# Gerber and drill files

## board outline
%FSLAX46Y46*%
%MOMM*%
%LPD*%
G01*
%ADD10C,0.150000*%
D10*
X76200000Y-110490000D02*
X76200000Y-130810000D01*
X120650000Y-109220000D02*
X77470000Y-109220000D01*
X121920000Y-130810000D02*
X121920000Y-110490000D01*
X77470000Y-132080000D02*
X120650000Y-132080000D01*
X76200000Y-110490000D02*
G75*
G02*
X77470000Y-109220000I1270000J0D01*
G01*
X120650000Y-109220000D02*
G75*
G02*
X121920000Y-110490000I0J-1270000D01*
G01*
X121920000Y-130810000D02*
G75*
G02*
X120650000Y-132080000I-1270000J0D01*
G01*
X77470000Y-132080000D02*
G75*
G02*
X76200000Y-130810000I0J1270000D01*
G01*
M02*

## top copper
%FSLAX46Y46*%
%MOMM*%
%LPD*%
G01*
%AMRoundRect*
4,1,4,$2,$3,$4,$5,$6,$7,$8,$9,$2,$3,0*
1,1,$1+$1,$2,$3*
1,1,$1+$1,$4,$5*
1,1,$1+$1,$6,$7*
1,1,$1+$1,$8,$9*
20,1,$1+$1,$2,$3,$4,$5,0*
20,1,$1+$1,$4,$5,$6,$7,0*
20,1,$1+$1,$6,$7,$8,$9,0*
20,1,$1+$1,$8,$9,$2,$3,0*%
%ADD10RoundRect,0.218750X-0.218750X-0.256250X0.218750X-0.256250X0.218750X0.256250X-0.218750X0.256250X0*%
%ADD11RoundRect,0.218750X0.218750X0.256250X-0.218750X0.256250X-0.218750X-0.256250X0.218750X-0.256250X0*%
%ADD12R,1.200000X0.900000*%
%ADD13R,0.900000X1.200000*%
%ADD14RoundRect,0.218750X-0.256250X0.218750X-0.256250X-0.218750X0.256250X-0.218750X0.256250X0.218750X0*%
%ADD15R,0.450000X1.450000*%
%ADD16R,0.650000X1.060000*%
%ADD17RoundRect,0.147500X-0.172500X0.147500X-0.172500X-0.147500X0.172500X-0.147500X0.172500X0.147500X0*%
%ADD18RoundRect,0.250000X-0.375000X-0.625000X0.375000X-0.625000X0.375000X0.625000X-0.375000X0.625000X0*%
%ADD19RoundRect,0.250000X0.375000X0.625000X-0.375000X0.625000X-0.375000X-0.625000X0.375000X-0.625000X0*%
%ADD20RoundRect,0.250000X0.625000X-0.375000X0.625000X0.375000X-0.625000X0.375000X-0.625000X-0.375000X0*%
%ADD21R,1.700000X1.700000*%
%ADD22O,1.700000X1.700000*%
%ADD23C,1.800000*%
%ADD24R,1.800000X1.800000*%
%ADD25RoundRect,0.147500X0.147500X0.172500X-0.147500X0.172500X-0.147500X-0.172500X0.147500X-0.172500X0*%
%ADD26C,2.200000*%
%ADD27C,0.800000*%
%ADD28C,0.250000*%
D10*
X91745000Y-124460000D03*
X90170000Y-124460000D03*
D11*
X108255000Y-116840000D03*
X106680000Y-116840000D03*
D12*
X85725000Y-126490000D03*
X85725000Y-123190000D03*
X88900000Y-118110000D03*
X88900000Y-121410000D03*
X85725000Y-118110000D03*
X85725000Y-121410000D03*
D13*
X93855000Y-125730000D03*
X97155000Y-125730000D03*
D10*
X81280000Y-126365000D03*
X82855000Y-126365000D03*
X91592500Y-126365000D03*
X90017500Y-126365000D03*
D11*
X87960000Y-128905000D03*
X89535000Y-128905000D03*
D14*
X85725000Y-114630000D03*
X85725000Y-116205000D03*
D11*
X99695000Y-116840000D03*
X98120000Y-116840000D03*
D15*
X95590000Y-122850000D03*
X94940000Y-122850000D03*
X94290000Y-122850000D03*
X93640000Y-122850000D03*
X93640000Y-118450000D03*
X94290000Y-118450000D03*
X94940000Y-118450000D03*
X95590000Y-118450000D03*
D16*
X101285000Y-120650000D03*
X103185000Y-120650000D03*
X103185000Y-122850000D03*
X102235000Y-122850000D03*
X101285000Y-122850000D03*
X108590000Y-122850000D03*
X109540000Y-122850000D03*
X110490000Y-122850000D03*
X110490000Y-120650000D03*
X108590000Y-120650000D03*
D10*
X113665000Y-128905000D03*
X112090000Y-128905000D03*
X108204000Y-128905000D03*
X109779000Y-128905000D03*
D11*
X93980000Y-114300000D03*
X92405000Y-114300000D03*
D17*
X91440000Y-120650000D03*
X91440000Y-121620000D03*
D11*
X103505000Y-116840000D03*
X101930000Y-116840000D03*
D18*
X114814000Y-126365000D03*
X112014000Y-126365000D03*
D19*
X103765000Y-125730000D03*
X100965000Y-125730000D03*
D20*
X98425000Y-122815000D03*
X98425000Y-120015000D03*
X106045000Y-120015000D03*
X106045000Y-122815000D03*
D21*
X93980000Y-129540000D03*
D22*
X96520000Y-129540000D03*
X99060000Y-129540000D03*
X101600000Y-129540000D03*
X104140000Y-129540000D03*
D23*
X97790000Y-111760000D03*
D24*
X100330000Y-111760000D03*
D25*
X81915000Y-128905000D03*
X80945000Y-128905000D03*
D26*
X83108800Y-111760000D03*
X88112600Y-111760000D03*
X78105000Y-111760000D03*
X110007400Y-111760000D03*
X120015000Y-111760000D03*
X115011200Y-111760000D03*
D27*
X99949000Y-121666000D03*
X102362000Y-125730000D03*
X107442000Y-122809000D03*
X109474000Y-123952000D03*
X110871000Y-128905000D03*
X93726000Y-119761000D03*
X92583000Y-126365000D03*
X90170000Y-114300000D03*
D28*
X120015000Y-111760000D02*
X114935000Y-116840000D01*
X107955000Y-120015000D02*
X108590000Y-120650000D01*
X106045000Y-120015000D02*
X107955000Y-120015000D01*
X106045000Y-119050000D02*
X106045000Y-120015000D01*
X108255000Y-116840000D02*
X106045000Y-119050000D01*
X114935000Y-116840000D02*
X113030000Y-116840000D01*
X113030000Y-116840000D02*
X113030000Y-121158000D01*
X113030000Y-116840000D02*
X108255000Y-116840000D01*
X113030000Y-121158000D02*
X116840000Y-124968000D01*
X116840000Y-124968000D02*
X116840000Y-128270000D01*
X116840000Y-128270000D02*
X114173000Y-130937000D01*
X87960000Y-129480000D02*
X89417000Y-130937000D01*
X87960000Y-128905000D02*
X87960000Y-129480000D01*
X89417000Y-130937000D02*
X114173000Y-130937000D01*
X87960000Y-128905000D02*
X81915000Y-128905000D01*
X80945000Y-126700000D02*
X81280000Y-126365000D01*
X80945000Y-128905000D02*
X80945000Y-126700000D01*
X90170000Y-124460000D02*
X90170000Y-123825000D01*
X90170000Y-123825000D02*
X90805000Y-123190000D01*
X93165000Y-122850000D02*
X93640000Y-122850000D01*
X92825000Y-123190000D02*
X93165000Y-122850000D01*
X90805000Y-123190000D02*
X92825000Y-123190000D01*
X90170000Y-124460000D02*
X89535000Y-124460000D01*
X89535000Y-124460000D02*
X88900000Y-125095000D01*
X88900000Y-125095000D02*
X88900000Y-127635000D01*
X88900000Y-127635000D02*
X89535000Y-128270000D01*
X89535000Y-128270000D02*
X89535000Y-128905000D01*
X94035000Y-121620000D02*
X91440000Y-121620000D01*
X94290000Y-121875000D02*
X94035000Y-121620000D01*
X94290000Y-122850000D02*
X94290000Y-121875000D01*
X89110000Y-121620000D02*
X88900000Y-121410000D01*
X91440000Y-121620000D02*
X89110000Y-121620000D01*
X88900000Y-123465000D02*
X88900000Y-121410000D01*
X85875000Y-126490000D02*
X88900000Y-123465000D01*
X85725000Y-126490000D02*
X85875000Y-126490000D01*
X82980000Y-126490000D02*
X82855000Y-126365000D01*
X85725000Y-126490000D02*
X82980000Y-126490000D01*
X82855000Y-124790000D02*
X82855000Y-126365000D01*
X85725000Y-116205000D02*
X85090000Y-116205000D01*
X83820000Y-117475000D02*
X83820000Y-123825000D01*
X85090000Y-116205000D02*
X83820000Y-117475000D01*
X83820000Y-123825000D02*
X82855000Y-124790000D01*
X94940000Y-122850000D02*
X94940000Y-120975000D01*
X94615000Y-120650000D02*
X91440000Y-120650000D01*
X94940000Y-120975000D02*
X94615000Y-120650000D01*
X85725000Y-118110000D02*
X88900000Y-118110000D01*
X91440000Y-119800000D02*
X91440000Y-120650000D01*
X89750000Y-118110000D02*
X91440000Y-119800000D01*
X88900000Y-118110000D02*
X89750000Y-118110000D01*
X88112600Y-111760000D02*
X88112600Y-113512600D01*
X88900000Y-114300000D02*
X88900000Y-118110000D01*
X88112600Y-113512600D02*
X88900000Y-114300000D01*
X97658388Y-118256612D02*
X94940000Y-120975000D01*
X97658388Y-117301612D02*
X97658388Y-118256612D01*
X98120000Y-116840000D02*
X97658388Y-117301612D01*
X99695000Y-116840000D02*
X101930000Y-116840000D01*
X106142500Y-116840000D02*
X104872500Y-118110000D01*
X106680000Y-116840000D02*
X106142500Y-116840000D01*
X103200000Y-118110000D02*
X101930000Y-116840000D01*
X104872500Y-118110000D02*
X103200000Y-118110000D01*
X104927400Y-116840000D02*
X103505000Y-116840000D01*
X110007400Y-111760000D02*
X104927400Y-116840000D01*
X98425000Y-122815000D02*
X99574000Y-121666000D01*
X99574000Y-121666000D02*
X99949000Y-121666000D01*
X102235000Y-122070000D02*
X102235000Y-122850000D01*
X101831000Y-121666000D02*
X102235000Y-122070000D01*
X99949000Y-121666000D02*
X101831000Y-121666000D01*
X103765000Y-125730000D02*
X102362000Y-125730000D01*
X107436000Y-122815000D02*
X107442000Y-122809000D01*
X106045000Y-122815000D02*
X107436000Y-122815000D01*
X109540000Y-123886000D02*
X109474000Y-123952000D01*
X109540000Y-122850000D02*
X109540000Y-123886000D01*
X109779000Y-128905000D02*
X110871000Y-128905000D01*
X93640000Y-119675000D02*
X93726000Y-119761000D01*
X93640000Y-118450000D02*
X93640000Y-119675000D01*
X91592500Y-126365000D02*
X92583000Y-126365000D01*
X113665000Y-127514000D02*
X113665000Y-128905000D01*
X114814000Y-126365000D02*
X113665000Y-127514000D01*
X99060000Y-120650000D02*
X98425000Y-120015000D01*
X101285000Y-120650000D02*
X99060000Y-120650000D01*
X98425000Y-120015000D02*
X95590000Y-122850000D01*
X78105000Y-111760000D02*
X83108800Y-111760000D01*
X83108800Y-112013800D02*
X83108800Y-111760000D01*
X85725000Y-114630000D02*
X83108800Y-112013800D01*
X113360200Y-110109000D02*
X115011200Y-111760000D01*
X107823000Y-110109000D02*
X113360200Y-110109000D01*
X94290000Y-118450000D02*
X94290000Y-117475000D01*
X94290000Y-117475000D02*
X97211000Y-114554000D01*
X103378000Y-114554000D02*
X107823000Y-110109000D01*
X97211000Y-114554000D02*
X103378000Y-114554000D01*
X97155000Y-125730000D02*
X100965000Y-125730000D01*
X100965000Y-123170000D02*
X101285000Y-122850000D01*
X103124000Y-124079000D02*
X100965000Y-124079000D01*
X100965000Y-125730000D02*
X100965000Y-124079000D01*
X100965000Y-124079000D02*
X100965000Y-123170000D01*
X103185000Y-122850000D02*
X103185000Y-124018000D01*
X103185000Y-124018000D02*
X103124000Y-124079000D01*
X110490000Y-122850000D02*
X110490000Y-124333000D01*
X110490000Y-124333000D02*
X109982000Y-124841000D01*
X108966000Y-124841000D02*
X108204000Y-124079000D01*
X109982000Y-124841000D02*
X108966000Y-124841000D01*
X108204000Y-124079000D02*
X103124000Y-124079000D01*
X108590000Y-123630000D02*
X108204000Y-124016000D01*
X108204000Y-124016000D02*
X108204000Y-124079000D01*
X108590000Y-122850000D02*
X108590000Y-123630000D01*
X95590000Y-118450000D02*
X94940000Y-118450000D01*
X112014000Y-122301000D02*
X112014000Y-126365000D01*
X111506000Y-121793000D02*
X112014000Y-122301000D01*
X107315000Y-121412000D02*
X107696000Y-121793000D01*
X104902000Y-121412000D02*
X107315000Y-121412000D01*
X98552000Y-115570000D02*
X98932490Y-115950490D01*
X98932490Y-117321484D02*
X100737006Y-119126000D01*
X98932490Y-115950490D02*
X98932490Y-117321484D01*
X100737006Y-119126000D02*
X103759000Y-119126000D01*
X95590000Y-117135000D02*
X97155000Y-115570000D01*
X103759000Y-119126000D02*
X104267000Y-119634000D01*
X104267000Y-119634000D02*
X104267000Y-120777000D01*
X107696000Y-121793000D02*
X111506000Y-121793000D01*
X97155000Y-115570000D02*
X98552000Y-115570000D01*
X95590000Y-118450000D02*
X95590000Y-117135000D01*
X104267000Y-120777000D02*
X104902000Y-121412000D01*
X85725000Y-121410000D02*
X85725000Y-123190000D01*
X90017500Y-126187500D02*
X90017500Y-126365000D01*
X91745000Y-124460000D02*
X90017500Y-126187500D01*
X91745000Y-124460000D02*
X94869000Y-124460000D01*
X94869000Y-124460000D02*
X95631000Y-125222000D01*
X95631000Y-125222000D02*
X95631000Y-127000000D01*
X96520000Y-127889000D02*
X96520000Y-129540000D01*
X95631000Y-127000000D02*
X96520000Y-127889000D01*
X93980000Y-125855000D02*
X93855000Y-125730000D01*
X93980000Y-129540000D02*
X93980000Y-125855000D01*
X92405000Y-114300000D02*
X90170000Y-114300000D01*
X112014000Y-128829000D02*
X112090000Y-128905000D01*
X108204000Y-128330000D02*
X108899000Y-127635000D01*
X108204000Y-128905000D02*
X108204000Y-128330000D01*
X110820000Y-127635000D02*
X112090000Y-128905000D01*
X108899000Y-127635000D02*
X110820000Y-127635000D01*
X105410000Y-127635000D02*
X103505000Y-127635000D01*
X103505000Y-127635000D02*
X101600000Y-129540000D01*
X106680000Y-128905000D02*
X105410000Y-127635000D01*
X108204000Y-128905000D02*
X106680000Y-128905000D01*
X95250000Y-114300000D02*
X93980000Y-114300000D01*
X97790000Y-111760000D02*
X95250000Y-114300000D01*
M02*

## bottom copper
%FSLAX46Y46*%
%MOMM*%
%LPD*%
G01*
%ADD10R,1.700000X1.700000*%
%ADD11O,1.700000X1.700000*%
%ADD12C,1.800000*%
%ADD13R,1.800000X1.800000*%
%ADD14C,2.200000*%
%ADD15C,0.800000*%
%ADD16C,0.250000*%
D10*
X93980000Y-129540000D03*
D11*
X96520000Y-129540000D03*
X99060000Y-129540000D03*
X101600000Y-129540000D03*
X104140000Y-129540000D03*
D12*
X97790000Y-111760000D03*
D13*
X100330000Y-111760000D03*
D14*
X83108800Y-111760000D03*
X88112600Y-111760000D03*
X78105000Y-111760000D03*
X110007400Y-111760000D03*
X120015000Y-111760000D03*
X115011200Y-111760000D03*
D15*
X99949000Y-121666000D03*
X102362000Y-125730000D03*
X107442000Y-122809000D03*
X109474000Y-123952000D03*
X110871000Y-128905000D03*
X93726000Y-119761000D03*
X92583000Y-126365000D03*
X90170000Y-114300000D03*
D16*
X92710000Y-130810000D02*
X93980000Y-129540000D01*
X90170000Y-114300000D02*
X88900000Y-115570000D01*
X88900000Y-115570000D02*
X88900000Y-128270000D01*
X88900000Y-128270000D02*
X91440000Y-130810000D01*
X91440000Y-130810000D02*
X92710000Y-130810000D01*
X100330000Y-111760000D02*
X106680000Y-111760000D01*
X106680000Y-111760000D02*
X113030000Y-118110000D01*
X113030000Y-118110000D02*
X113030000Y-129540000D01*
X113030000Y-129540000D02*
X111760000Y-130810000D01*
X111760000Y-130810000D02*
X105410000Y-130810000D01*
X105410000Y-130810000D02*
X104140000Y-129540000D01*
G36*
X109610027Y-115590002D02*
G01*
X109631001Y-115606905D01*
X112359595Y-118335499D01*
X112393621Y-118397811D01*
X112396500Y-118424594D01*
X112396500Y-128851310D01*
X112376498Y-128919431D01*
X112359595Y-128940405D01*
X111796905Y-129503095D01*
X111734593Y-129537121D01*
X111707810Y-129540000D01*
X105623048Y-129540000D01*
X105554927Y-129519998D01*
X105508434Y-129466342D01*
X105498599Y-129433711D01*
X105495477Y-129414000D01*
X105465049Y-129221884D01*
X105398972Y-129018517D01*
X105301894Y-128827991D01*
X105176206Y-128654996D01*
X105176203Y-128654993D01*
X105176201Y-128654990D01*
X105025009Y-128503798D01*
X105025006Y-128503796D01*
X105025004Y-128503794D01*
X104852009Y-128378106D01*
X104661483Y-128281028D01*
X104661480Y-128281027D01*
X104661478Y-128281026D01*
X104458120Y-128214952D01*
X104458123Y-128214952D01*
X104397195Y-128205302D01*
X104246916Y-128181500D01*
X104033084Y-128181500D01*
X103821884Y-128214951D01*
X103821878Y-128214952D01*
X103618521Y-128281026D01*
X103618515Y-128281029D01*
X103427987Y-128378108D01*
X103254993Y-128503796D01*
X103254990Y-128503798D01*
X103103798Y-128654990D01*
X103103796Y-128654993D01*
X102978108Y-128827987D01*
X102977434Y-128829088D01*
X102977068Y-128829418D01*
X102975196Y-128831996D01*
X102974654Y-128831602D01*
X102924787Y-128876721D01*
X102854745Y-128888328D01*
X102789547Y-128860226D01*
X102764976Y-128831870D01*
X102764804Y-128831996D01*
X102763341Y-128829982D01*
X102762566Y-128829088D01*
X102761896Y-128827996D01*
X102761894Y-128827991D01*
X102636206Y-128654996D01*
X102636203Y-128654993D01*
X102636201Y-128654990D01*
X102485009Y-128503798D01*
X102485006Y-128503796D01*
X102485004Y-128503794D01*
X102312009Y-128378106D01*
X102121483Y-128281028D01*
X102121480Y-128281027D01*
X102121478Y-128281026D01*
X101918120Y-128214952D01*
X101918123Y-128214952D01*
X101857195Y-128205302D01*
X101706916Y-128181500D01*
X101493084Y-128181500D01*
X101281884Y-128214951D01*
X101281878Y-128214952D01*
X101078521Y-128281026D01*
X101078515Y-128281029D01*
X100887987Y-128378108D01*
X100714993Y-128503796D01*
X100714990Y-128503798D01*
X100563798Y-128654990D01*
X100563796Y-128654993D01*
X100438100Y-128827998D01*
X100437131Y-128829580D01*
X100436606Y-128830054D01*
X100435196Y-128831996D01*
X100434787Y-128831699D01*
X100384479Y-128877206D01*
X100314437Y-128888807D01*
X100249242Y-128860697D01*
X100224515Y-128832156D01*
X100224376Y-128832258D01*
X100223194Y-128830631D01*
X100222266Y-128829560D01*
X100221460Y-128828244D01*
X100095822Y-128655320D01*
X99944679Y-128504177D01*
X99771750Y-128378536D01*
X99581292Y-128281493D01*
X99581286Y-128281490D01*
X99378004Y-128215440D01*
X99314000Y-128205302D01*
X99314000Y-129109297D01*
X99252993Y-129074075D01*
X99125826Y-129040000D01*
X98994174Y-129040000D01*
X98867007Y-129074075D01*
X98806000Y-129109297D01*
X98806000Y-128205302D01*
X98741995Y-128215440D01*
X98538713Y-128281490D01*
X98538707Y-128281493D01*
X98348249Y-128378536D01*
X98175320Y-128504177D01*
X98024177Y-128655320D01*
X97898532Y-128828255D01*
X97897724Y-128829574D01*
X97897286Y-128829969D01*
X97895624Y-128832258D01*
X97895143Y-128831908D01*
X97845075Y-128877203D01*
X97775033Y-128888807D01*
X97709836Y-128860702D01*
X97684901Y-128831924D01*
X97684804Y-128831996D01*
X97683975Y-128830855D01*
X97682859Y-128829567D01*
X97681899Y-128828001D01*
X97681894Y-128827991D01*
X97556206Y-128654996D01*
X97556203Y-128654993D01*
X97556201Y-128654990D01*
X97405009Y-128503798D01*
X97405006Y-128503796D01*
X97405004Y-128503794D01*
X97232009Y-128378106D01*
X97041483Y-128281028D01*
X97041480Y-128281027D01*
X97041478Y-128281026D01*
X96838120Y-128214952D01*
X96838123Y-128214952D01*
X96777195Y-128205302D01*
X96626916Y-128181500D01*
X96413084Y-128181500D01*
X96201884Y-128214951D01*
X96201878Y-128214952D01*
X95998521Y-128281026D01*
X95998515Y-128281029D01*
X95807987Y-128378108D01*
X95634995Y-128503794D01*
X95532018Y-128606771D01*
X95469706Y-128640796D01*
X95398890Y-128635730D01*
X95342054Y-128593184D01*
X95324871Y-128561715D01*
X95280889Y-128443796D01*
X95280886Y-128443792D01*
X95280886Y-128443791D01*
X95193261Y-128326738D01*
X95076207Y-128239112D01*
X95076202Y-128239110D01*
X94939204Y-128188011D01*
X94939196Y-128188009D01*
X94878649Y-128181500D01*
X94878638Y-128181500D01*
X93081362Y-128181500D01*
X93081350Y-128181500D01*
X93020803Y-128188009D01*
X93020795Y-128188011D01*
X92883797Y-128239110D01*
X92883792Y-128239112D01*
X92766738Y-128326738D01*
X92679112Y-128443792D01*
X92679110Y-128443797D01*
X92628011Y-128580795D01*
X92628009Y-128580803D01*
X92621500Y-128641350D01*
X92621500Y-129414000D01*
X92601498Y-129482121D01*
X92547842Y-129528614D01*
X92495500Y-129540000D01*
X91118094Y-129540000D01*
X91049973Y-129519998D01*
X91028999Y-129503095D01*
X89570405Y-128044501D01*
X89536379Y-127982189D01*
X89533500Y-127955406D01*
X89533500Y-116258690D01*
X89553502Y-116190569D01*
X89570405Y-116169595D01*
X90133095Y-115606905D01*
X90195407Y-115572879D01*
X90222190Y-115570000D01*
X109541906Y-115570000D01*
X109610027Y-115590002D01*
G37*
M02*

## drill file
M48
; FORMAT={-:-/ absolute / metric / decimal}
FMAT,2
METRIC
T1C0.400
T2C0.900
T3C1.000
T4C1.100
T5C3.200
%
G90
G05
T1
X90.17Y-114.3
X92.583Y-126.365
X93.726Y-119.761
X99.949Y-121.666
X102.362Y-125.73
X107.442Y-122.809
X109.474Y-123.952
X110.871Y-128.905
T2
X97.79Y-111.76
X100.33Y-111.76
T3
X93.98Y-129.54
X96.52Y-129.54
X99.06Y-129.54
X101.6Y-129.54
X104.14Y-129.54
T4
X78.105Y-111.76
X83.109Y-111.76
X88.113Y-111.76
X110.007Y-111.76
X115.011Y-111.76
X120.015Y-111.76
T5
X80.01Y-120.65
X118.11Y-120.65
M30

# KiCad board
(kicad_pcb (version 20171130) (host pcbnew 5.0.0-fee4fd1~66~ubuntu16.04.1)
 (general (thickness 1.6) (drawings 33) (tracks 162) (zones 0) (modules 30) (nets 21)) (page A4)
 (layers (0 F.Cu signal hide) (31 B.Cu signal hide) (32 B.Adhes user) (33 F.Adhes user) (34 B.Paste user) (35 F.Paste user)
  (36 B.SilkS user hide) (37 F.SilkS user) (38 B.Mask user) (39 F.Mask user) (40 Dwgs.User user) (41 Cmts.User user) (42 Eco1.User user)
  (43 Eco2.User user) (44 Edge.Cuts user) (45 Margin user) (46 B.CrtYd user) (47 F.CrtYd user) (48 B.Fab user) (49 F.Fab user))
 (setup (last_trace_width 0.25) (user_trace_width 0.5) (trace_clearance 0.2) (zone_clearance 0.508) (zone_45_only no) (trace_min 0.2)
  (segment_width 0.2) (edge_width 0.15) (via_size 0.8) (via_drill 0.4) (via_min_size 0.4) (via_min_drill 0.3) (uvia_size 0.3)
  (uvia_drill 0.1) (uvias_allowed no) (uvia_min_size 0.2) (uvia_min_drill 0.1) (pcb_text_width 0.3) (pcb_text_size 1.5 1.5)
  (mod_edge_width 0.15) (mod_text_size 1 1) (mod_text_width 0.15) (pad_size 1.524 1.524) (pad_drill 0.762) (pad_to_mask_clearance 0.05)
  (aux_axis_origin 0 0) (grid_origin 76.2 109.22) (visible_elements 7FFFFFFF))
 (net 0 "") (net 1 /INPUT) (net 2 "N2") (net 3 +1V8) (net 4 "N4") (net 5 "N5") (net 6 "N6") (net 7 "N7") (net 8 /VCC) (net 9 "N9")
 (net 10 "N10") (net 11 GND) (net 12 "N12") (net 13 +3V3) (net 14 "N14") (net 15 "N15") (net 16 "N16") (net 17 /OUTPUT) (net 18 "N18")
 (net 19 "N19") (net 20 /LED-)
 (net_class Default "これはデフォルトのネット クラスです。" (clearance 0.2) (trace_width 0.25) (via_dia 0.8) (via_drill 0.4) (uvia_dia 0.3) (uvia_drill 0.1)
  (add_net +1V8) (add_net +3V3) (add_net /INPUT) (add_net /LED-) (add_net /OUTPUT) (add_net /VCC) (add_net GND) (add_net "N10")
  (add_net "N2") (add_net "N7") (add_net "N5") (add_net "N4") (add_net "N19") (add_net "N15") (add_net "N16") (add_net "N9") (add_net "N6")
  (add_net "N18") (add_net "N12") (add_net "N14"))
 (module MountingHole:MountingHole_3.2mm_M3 (layer F.Cu) (at 80.01 120.65)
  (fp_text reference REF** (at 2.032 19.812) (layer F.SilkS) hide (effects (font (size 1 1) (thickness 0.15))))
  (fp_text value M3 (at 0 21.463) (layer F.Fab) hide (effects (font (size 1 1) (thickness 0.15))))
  (pad 1 np_thru_hole circle (at 0 0) (size 3.2 3.2) (drill 3.2) (layers *.Cu *.Mask)))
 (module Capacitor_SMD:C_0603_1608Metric (layer F.Cu) (at 90.9575 124.46)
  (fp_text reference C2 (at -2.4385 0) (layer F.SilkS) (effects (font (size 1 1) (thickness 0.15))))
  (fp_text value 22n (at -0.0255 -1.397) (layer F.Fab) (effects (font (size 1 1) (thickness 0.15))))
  (pad 2 smd roundrect (at 0.7875 0) (size 0.875 0.95) (layers F.Cu F.Paste F.Mask) (roundrect_rratio 0.25) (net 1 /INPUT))
  (pad 1 smd roundrect (at -0.7875 0) (size 0.875 0.95) (layers F.Cu F.Paste F.Mask) (roundrect_rratio 0.25) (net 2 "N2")))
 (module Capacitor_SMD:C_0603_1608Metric (layer F.Cu) (at 107.4675 116.84 180)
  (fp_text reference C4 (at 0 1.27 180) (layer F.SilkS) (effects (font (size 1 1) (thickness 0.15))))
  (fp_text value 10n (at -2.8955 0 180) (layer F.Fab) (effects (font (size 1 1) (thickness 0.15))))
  (pad 1 smd roundrect (at -0.7875 0 180) (size 0.875 0.95) (layers F.Cu F.Paste F.Mask) (roundrect_rratio 0.25) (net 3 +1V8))
  (pad 2 smd roundrect (at 0.7875 0 180) (size 0.875 0.95) (layers F.Cu F.Paste F.Mask) (roundrect_rratio 0.25) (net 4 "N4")))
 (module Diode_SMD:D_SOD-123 (layer F.Cu) (at 85.725 124.84 90)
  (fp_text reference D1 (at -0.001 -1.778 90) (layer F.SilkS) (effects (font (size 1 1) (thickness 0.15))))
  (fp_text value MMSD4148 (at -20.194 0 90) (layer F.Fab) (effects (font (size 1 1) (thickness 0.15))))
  (pad 1 smd rect (at -1.65 0 90) (size 0.9 1.2) (layers F.Cu F.Paste F.Mask) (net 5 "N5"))
  (pad 2 smd rect (at 1.65 0 90) (size 0.9 1.2) (layers F.Cu F.Paste F.Mask) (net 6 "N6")))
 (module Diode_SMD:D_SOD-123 (layer F.Cu) (at 88.9 119.76 270)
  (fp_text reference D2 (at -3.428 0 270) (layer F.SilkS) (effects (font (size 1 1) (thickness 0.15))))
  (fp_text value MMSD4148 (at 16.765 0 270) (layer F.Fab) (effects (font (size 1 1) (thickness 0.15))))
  (pad 1 smd rect (at -1.65 0 270) (size 0.9 1.2) (layers F.Cu F.Paste F.Mask) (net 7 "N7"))
  (pad 2 smd rect (at 1.65 0 270) (size 0.9 1.2) (layers F.Cu F.Paste F.Mask) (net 5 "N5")))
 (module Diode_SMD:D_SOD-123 (layer F.Cu) (at 85.725 119.76 90)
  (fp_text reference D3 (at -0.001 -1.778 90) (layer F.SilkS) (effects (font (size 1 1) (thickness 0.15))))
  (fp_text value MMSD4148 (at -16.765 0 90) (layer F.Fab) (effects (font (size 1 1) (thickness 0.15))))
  (pad 2 smd rect (at 1.65 0 90) (size 0.9 1.2) (layers F.Cu F.Paste F.Mask) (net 7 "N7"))
  (pad 1 smd rect (at -1.65 0 90) (size 0.9 1.2) (layers F.Cu F.Paste F.Mask) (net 6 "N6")))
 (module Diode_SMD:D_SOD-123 (layer F.Cu) (at 95.505 125.73 180)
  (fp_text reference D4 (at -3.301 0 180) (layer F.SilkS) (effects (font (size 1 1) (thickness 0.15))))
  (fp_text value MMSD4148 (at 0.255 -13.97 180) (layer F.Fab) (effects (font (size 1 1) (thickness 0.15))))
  (pad 2 smd rect (at 1.65 0 180) (size 0.9 1.2) (layers F.Cu F.Paste F.Mask) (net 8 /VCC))
  (pad 1 smd rect (at -1.65 0 180) (size 0.9 1.2) (layers F.Cu F.Paste F.Mask) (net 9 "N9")))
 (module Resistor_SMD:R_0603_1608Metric (layer F.Cu) (at 82.0675 126.365)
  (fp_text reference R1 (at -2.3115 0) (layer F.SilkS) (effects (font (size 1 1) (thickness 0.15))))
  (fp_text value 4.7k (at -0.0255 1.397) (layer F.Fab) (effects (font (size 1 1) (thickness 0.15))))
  (pad 1 smd roundrect (at -0.7875 0) (size 0.875 0.95) (layers F.Cu F.Paste F.Mask) (roundrect_rratio 0.25) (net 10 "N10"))
  (pad 2 smd roundrect (at 0.7875 0) (size 0.875 0.95) (layers F.Cu F.Paste F.Mask) (roundrect_rratio 0.25) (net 5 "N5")))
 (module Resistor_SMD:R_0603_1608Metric (layer F.Cu) (at 90.805 126.365)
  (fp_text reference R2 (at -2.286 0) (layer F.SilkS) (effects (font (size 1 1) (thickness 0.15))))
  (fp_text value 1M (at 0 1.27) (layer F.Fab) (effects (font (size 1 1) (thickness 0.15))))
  (pad 2 smd roundrect (at 0.7875 0) (size 0.875 0.95) (layers F.Cu F.Paste F.Mask) (roundrect_rratio 0.25) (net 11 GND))
  (pad 1 smd roundrect (at -0.7875 0) (size 0.875 0.95) (layers F.Cu F.Paste F.Mask) (roundrect_rratio 0.25) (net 1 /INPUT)))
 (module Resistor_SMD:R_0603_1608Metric (layer F.Cu) (at 88.7475 128.905 180)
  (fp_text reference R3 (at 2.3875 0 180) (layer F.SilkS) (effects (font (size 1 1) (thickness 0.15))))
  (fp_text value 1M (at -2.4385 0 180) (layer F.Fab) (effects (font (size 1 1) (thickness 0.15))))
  (pad 2 smd roundrect (at 0.7875 0 180) (size 0.875 0.95) (layers F.Cu F.Paste F.Mask) (roundrect_rratio 0.25) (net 3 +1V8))
  (pad 1 smd roundrect (at -0.7875 0 180) (size 0.875 0.95) (layers F.Cu F.Paste F.Mask) (roundrect_rratio 0.25) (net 2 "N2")))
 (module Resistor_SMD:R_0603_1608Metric (layer F.Cu) (at 85.725 115.4175 270)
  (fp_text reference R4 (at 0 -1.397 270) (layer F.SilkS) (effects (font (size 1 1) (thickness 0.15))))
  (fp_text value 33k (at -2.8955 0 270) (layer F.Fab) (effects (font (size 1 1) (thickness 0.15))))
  (pad 1 smd roundrect (at -0.7875 0 270) (size 0.875 0.95) (layers F.Cu F.Paste F.Mask) (roundrect_rratio 0.25) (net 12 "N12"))
  (pad 2 smd roundrect (at 0.7875 0 270) (size 0.875 0.95) (layers F.Cu F.Paste F.Mask) (roundrect_rratio 0.25) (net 5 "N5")))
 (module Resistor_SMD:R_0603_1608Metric (layer F.Cu) (at 98.9075 116.84 180)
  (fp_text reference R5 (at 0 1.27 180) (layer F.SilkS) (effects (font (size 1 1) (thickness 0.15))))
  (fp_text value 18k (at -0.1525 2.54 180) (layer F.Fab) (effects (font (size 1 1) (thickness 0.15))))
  (pad 1 smd roundrect (at -0.7875 0 180) (size 0.875 0.95) (layers F.Cu F.Paste F.Mask) (roundrect_rratio 0.25) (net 4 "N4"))
  (pad 2 smd roundrect (at 0.7875 0 180) (size 0.875 0.95) (layers F.Cu F.Paste F.Mask) (roundrect_rratio 0.25) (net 7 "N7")))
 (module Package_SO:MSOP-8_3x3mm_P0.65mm (layer F.Cu) (at 94.615 120.65 270)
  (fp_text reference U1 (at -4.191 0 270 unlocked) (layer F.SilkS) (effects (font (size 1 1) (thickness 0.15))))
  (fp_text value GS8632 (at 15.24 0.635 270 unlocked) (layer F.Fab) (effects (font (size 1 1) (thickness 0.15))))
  (pad 8 smd rect (at 2.2 -0.975 270) (size 1.45 0.45) (layers F.Cu F.Paste F.Mask) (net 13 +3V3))
  (pad 7 smd rect (at 2.2 -0.325 270) (size 1.45 0.45) (layers F.Cu F.Paste F.Mask) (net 7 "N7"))
  (pad 6 smd rect (at 2.2 0.325 270) (size 1.45 0.45) (layers F.Cu F.Paste F.Mask) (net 5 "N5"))
  (pad 5 smd rect (at 2.2 0.975 270) (size 1.45 0.45) (layers F.Cu F.Paste F.Mask) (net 2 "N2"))
  (pad 4 smd rect (at -2.2 0.975 270) (size 1.45 0.45) (layers F.Cu F.Paste F.Mask) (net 11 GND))
  (pad 3 smd rect (at -2.2 0.325 270) (size 1.45 0.45) (layers F.Cu F.Paste F.Mask) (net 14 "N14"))
  (pad 2 smd rect (at -2.2 -0.325 270) (size 1.45 0.45) (layers F.Cu F.Paste F.Mask) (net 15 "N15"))
  (pad 1 smd rect (at -2.2 -0.975 270) (size 1.45 0.45) (layers F.Cu F.Paste F.Mask) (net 15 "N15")))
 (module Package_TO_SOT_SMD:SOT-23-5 (layer F.Cu) (at 102.235 121.75 90)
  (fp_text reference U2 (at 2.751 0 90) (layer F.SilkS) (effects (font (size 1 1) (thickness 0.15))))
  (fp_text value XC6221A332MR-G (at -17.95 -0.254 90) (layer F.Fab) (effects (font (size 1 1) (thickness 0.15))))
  (pad 5 smd rect (at 1.1 -0.95 90) (size 1.06 0.65) (layers F.Cu F.Paste F.Mask) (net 13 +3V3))
  (pad 4 smd rect (at 1.1 0.95 90) (size 1.06 0.65) (layers F.Cu F.Paste F.Mask))
  (pad 3 smd rect (at -1.1 0.95 90) (size 1.06 0.65) (layers F.Cu F.Paste F.Mask) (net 9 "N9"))
  (pad 2 smd rect (at -1.1 0 90) (size 1.06 0.65) (layers F.Cu F.Paste F.Mask) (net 11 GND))
  (pad 1 smd rect (at -1.1 -0.95 90) (size 1.06 0.65) (layers F.Cu F.Paste F.Mask) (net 9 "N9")))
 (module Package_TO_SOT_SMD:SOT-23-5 (layer F.Cu) (at 109.54 121.75 90)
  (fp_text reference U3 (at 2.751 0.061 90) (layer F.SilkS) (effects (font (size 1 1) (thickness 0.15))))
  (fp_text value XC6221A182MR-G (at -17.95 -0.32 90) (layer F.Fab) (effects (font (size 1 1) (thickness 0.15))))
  (pad 1 smd rect (at -1.1 -0.95 90) (size 1.06 0.65) (layers F.Cu F.Paste F.Mask) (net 9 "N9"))
  (pad 2 smd rect (at -1.1 0 90) (size 1.06 0.65) (layers F.Cu F.Paste F.Mask) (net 11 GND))
  (pad 3 smd rect (at -1.1 0.95 90) (size 1.06 0.65) (layers F.Cu F.Paste F.Mask) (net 9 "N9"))
  (pad 4 smd rect (at 1.1 0.95 90) (size 1.06 0.65) (layers F.Cu F.Paste F.Mask))
  (pad 5 smd rect (at 1.1 -0.95 90) (size 1.06 0.65) (layers F.Cu F.Paste F.Mask) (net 3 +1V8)))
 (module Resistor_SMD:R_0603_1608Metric (layer F.Cu) (at 112.8775 128.905)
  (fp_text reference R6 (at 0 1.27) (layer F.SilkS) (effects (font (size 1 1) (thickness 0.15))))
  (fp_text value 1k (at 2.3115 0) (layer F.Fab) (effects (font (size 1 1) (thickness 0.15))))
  (pad 2 smd roundrect (at 0.7875 0) (size 0.875 0.95) (layers F.Cu F.Paste F.Mask) (roundrect_rratio 0.25) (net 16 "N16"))
  (pad 1 smd roundrect (at -0.7875 0) (size 0.875 0.95) (layers F.Cu F.Paste F.Mask) (roundrect_rratio 0.25) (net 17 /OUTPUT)))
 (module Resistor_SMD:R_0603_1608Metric (layer F.Cu) (at 108.9915 128.905)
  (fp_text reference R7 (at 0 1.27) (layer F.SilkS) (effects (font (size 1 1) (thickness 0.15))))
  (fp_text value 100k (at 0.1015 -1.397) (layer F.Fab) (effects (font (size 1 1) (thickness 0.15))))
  (pad 1 smd roundrect (at -0.7875 0) (size 0.875 0.95) (layers F.Cu F.Paste F.Mask) (roundrect_rratio 0.25) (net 17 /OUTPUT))
  (pad 2 smd roundrect (at 0.7875 0) (size 0.875 0.95) (layers F.Cu F.Paste F.Mask) (roundrect_rratio 0.25) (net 11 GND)))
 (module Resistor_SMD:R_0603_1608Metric (layer F.Cu) (at 93.1925 114.3 180)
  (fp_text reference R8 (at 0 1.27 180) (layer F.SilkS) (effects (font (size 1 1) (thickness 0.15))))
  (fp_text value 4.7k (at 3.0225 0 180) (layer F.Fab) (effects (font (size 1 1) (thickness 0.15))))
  (pad 1 smd roundrect (at -0.7875 0 180) (size 0.875 0.95) (layers F.Cu F.Paste F.Mask) (roundrect_rratio 0.25) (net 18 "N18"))
  (pad 2 smd roundrect (at 0.7875 0 180) (size 0.875 0.95) (layers F.Cu F.Paste F.Mask) (roundrect_rratio 0.25) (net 8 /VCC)))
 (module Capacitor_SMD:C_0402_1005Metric (layer F.Cu) (at 91.44 121.135 270)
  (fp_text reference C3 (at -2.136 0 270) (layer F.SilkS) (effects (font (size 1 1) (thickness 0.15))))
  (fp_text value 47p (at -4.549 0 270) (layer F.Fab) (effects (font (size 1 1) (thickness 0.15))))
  (pad 1 smd roundrect (at -0.485 0 270) (size 0.59 0.64) (layers F.Cu F.Paste F.Mask) (roundrect_rratio 0.25) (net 7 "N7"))
  (pad 2 smd roundrect (at 0.485 0 270) (size 0.59 0.64) (layers F.Cu F.Paste F.Mask) (roundrect_rratio 0.25) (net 5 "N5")))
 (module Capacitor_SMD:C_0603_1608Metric (layer F.Cu) (at 102.7175 116.84 180)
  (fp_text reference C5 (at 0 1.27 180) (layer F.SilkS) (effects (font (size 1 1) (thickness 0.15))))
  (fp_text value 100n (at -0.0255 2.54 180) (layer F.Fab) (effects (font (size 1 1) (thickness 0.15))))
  (pad 1 smd roundrect (at -0.7875 0 180) (size 0.875 0.95) (layers F.Cu F.Paste F.Mask) (roundrect_rratio 0.25) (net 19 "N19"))
  (pad 2 smd roundrect (at 0.7875 0 180) (size 0.875 0.95) (layers F.Cu F.Paste F.Mask) (roundrect_rratio 0.25) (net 4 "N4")))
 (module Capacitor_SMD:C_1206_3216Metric (layer F.Cu) (at 113.414 126.365)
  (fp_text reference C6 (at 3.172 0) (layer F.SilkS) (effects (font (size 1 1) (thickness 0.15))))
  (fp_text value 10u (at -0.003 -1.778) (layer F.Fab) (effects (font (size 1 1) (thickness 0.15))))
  (pad 2 smd roundrect (at 1.4 0) (size 1.25 1.75) (layers F.Cu F.Paste F.Mask) (roundrect_rratio 0.2) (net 16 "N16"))
  (pad 1 smd roundrect (at -1.4 0) (size 1.25 1.75) (layers F.Cu F.Paste F.Mask) (roundrect_rratio 0.2) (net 15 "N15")))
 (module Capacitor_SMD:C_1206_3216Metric (layer F.Cu) (at 102.365 125.73 180)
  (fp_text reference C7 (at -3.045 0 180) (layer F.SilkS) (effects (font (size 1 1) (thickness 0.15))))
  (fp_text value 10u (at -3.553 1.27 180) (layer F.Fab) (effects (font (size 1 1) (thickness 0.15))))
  (pad 1 smd roundrect (at -1.4 0 180) (size 1.25 1.75) (layers F.Cu F.Paste F.Mask) (roundrect_rratio 0.2) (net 11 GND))
  (pad 2 smd roundrect (at 1.4 0 180) (size 1.25 1.75) (layers F.Cu F.Paste F.Mask) (roundrect_rratio 0.2) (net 9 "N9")))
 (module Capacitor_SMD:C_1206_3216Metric (layer F.Cu) (at 98.425 121.415 90)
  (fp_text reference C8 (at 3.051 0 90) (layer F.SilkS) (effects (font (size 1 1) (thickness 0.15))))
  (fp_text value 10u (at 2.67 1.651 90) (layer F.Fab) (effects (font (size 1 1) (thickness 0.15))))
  (pad 1 smd roundrect (at -1.4 0 90) (size 1.25 1.75) (layers F.Cu F.Paste F.Mask) (roundrect_rratio 0.2) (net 11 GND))
  (pad 2 smd roundrect (at 1.4 0 90) (size 1.25 1.75) (layers F.Cu F.Paste F.Mask) (roundrect_rratio 0.2) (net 13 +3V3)))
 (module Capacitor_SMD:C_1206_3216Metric (layer F.Cu) (at 106.045 121.415 90)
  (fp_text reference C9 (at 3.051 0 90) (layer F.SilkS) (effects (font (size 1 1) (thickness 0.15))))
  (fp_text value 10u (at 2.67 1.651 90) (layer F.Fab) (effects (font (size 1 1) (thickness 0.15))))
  (pad 2 smd roundrect (at 1.4 0 90) (size 1.25 1.75) (layers F.Cu F.Paste F.Mask) (roundrect_rratio 0.2) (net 3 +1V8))
  (pad 1 smd roundrect (at -1.4 0 90) (size 1.25 1.75) (layers F.Cu F.Paste F.Mask) (roundrect_rratio 0.2) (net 11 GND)))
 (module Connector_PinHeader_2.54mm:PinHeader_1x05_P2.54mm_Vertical (layer F.Cu) (at 93.98 129.54 90)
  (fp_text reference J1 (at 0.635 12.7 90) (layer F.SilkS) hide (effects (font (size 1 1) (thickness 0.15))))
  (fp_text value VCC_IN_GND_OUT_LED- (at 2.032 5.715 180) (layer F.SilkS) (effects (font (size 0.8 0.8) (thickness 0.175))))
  (pad 1 thru_hole rect (at 0 0 90) (size 1.7 1.7) (drill 1) (layers *.Cu *.Mask) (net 8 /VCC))
  (pad 2 thru_hole oval (at 0 2.54 90) (size 1.7 1.7) (drill 1) (layers *.Cu *.Mask) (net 1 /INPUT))
  (pad 3 thru_hole oval (at 0 5.08 90) (size 1.7 1.7) (drill 1) (layers *.Cu *.Mask) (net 11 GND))
  (pad 4 thru_hole oval (at 0 7.62 90) (size 1.7 1.7) (drill 1) (layers *.Cu *.Mask) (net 17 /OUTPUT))
  (pad 5 thru_hole oval (at 0 10.16 90) (size 1.7 1.7) (drill 1) (layers *.Cu *.Mask) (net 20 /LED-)))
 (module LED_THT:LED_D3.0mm (layer F.Cu) (at 100.33 111.76 180)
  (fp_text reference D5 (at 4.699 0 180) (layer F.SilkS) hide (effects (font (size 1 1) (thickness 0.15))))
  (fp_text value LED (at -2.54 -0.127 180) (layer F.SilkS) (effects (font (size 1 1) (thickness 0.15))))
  (pad 2 thru_hole circle (at 2.54 0 180) (size 1.8 1.8) (drill 0.9) (layers *.Cu *.Mask) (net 18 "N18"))
  (pad 1 thru_hole rect (at 0 0 180) (size 1.8 1.8) (drill 0.9) (layers *.Cu *.Mask) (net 20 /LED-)))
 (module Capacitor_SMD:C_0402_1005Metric (layer F.Cu) (at 81.43 128.905 180)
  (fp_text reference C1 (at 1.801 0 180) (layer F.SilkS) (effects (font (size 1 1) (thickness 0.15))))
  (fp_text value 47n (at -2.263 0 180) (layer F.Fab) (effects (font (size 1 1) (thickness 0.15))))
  (pad 1 smd roundrect (at -0.485 0 180) (size 0.59 0.64) (layers F.Cu F.Paste F.Mask) (roundrect_rratio 0.25) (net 3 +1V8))
  (pad 2 smd roundrect (at 0.485 0 180) (size 0.59 0.64) (layers F.Cu F.Paste F.Mask) (roundrect_rratio 0.25) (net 10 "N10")))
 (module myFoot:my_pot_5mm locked (layer F.Cu) (at 83.1088 111.76 180)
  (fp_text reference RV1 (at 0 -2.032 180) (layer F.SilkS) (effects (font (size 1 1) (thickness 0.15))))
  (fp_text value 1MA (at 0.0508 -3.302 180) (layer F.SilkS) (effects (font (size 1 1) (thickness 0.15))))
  (pad 2 thru_hole circle (at 0 0 180) (size 2.2 2.2) (drill 1.1) (layers *.Cu *.Mask) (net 12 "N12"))
  (pad 1 thru_hole circle (at -5.0038 0 180) (size 2.2 2.2) (drill 1.1) (layers *.Cu *.Mask) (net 7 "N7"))
  (pad 3 thru_hole circle (at 5.0038 0 180) (size 2.2 2.2) (drill 1.1) (layers *.Cu *.Mask) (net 12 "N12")))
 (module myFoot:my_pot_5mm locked (layer F.Cu) (at 115.0112 111.76 180)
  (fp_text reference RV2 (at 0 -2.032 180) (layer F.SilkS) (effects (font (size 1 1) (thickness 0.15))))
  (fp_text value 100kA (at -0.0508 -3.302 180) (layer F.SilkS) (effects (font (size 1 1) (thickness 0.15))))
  (pad 3 thru_hole circle (at 5.0038 0 180) (size 2.2 2.2) (drill 1.1) (layers *.Cu *.Mask) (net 19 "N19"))
  (pad 1 thru_hole circle (at -5.0038 0 180) (size 2.2 2.2) (drill 1.1) (layers *.Cu *.Mask) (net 3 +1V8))
  (pad 2 thru_hole circle (at 0 0 180) (size 2.2 2.2) (drill 1.1) (layers *.Cu *.Mask) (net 14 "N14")))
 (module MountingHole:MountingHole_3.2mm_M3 (layer F.Cu) (at 118.11 120.65)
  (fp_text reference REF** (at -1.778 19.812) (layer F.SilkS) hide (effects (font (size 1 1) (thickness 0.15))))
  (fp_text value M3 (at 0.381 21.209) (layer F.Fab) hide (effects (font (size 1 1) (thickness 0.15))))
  (pad 1 np_thru_hole circle (at 0 0) (size 3.2 3.2) (drill 3.2) (layers *.Cu *.Mask)))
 (gr_line (start 76.2 110.49) (end 76.2 130.81) (layer Edge.Cuts) (width 0.15))
 (gr_line (start 120.65 109.22) (end 77.47 109.22) (layer Edge.Cuts) (width 0.15))
 (gr_line (start 121.92 130.81) (end 121.92 110.49) (layer Edge.Cuts) (width 0.15))
 (gr_line (start 77.47 132.08) (end 120.65 132.08) (layer Edge.Cuts) (width 0.15))
 (gr_arc (start 77.47 110.49) (end 77.47 109.22) (angle -90) (layer Edge.Cuts) (width 0.15))
 (gr_arc (start 120.65 110.49) (end 121.92 110.49) (angle -90) (layer Edge.Cuts) (width 0.15))
 (gr_arc (start 120.65 130.81) (end 120.65 132.08) (angle -90) (layer Edge.Cuts) (width 0.15))
 (gr_arc (start 77.47 130.81) (end 76.2 130.81) (angle -90) (layer Edge.Cuts) (width 0.15))
 (segment (start 120.015 111.76) (end 114.935 116.84) (width 0.25) (layer F.Cu) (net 3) (status 10))
 (segment (start 107.955 120.015) (end 108.59 120.65) (width 0.25) (layer F.Cu) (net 3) (status 20))
 (segment (start 106.045 120.015) (end 107.955 120.015) (width 0.25) (layer F.Cu) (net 3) (status 10))
 (segment (start 106.045 119.05) (end 106.045 120.015) (width 0.25) (layer F.Cu) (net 3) (status 20))
 (segment (start 108.255 116.84) (end 106.045 119.05) (width 0.25) (layer F.Cu) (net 3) (status 10))
 (segment (start 114.935 116.84) (end 113.03 116.84) (width 0.25) (layer F.Cu) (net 3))
 (segment (start 113.03 116.84) (end 113.03 121.158) (width 0.25) (layer F.Cu) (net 3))
 (segment (start 113.03 116.84) (end 108.255 116.84) (width 0.25) (layer F.Cu) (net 3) (status 20))
 (segment (start 113.03 121.158) (end 116.84 124.968) (width 0.25) (layer F.Cu) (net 3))
 (segment (start 116.84 124.968) (end 116.84 128.27) (width 0.25) (layer F.Cu) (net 3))
 (segment (start 116.84 128.27) (end 114.173 130.937) (width 0.25) (layer F.Cu) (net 3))
 (segment (start 87.96 129.48) (end 89.417 130.937) (width 0.25) (layer F.Cu) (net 3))
 (segment (start 87.96 128.905) (end 87.96 129.48) (width 0.25) (layer F.Cu) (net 3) (status 10))
 (segment (start 89.417 130.937) (end 114.173 130.937) (width 0.25) (layer F.Cu) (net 3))
 (segment (start 87.96 128.905) (end 81.915 128.905) (width 0.25) (layer F.Cu) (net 3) (status 30))
 (segment (start 80.945 126.7) (end 81.28 126.365) (width 0.25) (layer F.Cu) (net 10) (status 30))
 (segment (start 80.945 128.905) (end 80.945 126.7) (width 0.25) (layer F.Cu) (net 10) (status 30))
 (segment (start 90.17 124.46) (end 90.17 123.825) (width 0.25) (layer F.Cu) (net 2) (status 10))
 (segment (start 90.17 123.825) (end 90.805 123.19) (width 0.25) (layer F.Cu) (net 2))
 (segment (start 93.165 122.85) (end 93.64 122.85) (width 0.25) (layer F.Cu) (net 2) (status 20))
 (segment (start 92.825 123.19) (end 93.165 122.85) (width 0.25) (layer F.Cu) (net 2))
 (segment (start 90.805 123.19) (end 92.825 123.19) (width 0.25) (layer F.Cu) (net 2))
 (segment (start 90.17 124.46) (end 89.535 124.46) (width 0.25) (layer F.Cu) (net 2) (status 10))
 (segment (start 89.535 124.46) (end 88.9 125.095) (width 0.25) (layer F.Cu) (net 2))
 (segment (start 88.9 125.095) (end 88.9 127.635) (width 0.25) (layer F.Cu) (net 2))
 (segment (start 88.9 127.635) (end 89.535 128.27) (width 0.25) (layer F.Cu) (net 2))
 (segment (start 89.535 128.27) (end 89.535 128.905) (width 0.25) (layer F.Cu) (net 2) (status 20))
 (segment (start 94.035 121.62) (end 91.44 121.62) (width 0.25) (layer F.Cu) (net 5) (status 20))
 (segment (start 94.29 121.875) (end 94.035 121.62) (width 0.25) (layer F.Cu) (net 5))
 (segment (start 94.29 122.85) (end 94.29 121.875) (width 0.25) (layer F.Cu) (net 5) (status 10))
 (segment (start 89.11 121.62) (end 88.9 121.41) (width 0.25) (layer F.Cu) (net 5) (status 30))
 (segment (start 91.44 121.62) (end 89.11 121.62) (width 0.25) (layer F.Cu) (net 5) (status 30))
 (segment (start 88.9 123.465) (end 88.9 121.41) (width 0.25) (layer F.Cu) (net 5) (status 20))
 (segment (start 85.875 126.49) (end 88.9 123.465) (width 0.25) (layer F.Cu) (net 5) (status 10))
 (segment (start 85.725 126.49) (end 85.875 126.49) (width 0.25) (layer F.Cu) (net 5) (status 30))
 (segment (start 82.98 126.49) (end 82.855 126.365) (width 0.25) (layer F.Cu) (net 5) (status 30))
 (segment (start 85.725 126.49) (end 82.98 126.49) (width 0.25) (layer F.Cu) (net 5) (status 30))
 (segment (start 82.855 124.79) (end 82.855 126.365) (width 0.25) (layer F.Cu) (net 5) (status 20))
 (segment (start 85.725 116.205) (end 85.09 116.205) (width 0.25) (layer F.Cu) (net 5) (status 10))
 (segment (start 83.82 117.475) (end 83.82 123.825) (width 0.25) (layer F.Cu) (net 5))
 (segment (start 85.09 116.205) (end 83.82 117.475) (width 0.25) (layer F.Cu) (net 5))
 (segment (start 83.82 123.825) (end 82.855 124.79) (width 0.25) (layer F.Cu) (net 5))
 (segment (start 94.94 122.85) (end 94.94 120.975) (width 0.25) (layer F.Cu) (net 7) (status 10))
 (segment (start 94.615 120.65) (end 91.44 120.65) (width 0.25) (layer F.Cu) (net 7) (status 20))
 (segment (start 94.94 120.975) (end 94.615 120.65) (width 0.25) (layer F.Cu) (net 7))
 (segment (start 85.725 118.11) (end 88.9 118.11) (width 0.25) (layer F.Cu) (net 7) (status 30))
 (segment (start 91.44 119.8) (end 91.44 120.65) (width 0.25) (layer F.Cu) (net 7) (status 20))
 (segment (start 89.75 118.11) (end 91.44 119.8) (width 0.25) (layer F.Cu) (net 7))
 (segment (start 88.9 118.11) (end 89.75 118.11) (width 0.25) (layer F.Cu) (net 7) (status 10))
 (segment (start 88.1126 111.76) (end 88.1126 113.5126) (width 0.25) (layer F.Cu) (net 7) (status 10))
 (segment (start 88.9 114.3) (end 88.9 118.11) (width 0.25) (layer F.Cu) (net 7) (status 20))
 (segment (start 88.1126 113.5126) (end 88.9 114.3) (width 0.25) (layer F.Cu) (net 7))
 (segment (start 97.658388 118.256612) (end 94.94 120.975) (width 0.25) (layer F.Cu) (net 7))
 (segment (start 97.658388 117.301612) (end 97.658388 118.256612) (width 0.25) (layer F.Cu) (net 7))
 (segment (start 98.12 116.84) (end 97.658388 117.301612) (width 0.25) (layer F.Cu) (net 7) (status 10))
 (segment (start 99.695 116.84) (end 101.93 116.84) (width 0.25) (layer F.Cu) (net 4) (status 30))
 (segment (start 106.1425 116.84) (end 104.8725 118.11) (width 0.25) (layer F.Cu) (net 4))
 (segment (start 106.68 116.84) (end 106.1425 116.84) (width 0.25) (layer F.Cu) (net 4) (status 10))
 (segment (start 103.2 118.11) (end 101.93 116.84) (width 0.25) (layer F.Cu) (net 4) (status 20))
 (segment (start 104.8725 118.11) (end 103.2 118.11) (width 0.25) (layer F.Cu) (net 4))
 (segment (start 104.9274 116.84) (end 103.505 116.84) (width 0.25) (layer F.Cu) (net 19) (status 20))
 (segment (start 110.0074 111.76) (end 104.9274 116.84) (width 0.25) (layer F.Cu) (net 19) (status 10))
 (segment (start 98.425 122.815) (end 99.574 121.666) (width 0.25) (layer F.Cu) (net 11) (status 10))
 (via (at 99.949 121.666) (size 0.8) (drill 0.4) (layers F.Cu B.Cu) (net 11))
 (segment (start 99.574 121.666) (end 99.949 121.666) (width 0.25) (layer F.Cu) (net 11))
 (segment (start 102.235 122.07) (end 102.235 122.85) (width 0.25) (layer F.Cu) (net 11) (status 20))
 (segment (start 101.831 121.666) (end 102.235 122.07) (width 0.25) (layer F.Cu) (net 11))
 (segment (start 99.949 121.666) (end 101.831 121.666) (width 0.25) (layer F.Cu) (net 11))
 (via (at 102.362 125.73) (size 0.8) (drill 0.4) (layers F.Cu B.Cu) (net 11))
 (segment (start 103.765 125.73) (end 102.362 125.73) (width 0.25) (layer F.Cu) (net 11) (status 10))
 (via (at 107.442 122.809) (size 0.8) (drill 0.4) (layers F.Cu B.Cu) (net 11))
 (segment (start 107.436 122.815) (end 107.442 122.809) (width 0.25) (layer F.Cu) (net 11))
 (segment (start 106.045 122.815) (end 107.436 122.815) (width 0.25) (layer F.Cu) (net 11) (status 10))
 (via (at 109.474 123.952) (size 0.8) (drill 0.4) (layers F.Cu B.Cu) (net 11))
 (segment (start 109.54 123.886) (end 109.474 123.952) (width 0.25) (layer F.Cu) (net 11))
 (segment (start 109.54 122.85) (end 109.54 123.886) (width 0.25) (layer F.Cu) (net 11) (status 10))
 (via (at 110.871 128.905) (size 0.8) (drill 0.4) (layers F.Cu B.Cu) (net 11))
 (segment (start 109.779 128.905) (end 110.871 128.905) (width 0.25) (layer F.Cu) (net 11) (status 10))
 (via (at 93.726 119.761) (size 0.8) (drill 0.4) (layers F.Cu B.Cu) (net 11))
 (segment (start 93.64 119.675) (end 93.726 119.761) (width 0.25) (layer F.Cu) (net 11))
 (segment (start 93.64 118.45) (end 93.64 119.675) (width 0.25) (layer F.Cu) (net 11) (status 10))
 (via (at 92.583 126.365) (size 0.8) (drill 0.4) (layers F.Cu B.Cu) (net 11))
 (segment (start 91.5925 126.365) (end 92.583 126.365) (width 0.25) (layer F.Cu) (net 11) (status 10))
 (segment (start 113.665 127.514) (end 113.665 128.905) (width 0.25) (layer F.Cu) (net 16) (status 20))
 (segment (start 114.814 126.365) (end 113.665 127.514) (width 0.25) (layer F.Cu) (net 16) (status 10))
 (segment (start 99.06 120.65) (end 98.425 120.015) (width 0.25) (layer F.Cu) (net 13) (status 20))
 (segment (start 101.285 120.65) (end 99.06 120.65) (width 0.25) (layer F.Cu) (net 13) (status 10))
 (segment (start 98.425 120.015) (end 95.59 122.85) (width 0.25) (layer F.Cu) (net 13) (status 30))
 (segment (start 78.105 111.76) (end 83.1088 111.76) (width 0.25) (layer F.Cu) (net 12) (status 30))
 (segment (start 83.1088 112.0138) (end 83.1088 111.76) (width 0.25) (layer F.Cu) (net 12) (status 30))
 (segment (start 85.725 114.63) (end 83.1088 112.0138) (width 0.25) (layer F.Cu) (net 12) (status 30))
 (segment (start 113.3602 110.109) (end 115.0112 111.76) (width 0.25) (layer F.Cu) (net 14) (status 20))
 (segment (start 107.823 110.109) (end 113.3602 110.109) (width 0.25) (layer F.Cu) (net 14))
 (segment (start 94.29 118.45) (end 94.29 117.475) (width 0.25) (layer F.Cu) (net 14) (status 10))
 (segment (start 94.29 117.475) (end 97.211 114.554) (width 0.25) (layer F.Cu) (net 14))
 (segment (start 103.378 114.554) (end 107.823 110.109) (width 0.25) (layer F.Cu) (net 14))
 (segment (start 97.211 114.554) (end 103.378 114.554) (width 0.25) (layer F.Cu) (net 14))
 (segment (start 97.155 125.73) (end 100.965 125.73) (width 0.25) (layer F.Cu) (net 9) (status 30))
 (segment (start 100.965 123.17) (end 101.285 122.85) (width 0.25) (layer F.Cu) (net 9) (status 30))
 (segment (start 103.124 124.079) (end 100.965 124.079) (width 0.25) (layer F.Cu) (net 9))
 (segment (start 100.965 125.73) (end 100.965 124.079) (width 0.25) (layer F.Cu) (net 9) (status 10))
 (segment (start 100.965 124.079) (end 100.965 123.17) (width 0.25) (layer F.Cu) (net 9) (status 20))
 (segment (start 103.185 122.85) (end 103.185 124.018) (width 0.25) (layer F.Cu) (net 9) (status 10))
 (segment (start 103.185 124.018) (end 103.124 124.079) (width 0.25) (layer F.Cu) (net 9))
 (segment (start 110.49 122.85) (end 110.49 124.333) (width 0.25) (layer F.Cu) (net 9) (status 10))
 (segment (start 110.49 124.333) (end 109.982 124.841) (width 0.25) (layer F.Cu) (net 9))
 (segment (start 108.966 124.841) (end 108.204 124.079) (width 0.25) (layer F.Cu) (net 9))
 (segment (start 109.982 124.841) (end 108.966 124.841) (width 0.25) (layer F.Cu) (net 9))
 (segment (start 108.204 124.079) (end 103.124 124.079) (width 0.25) (layer F.Cu) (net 9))
 (segment (start 108.59 123.63) (end 108.204 124.016) (width 0.25) (layer F.Cu) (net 9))
 (segment (start 108.204 124.016) (end 108.204 124.079) (width 0.25) (layer F.Cu) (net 9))
 (segment (start 108.59 122.85) (end 108.59 123.63) (width 0.25) (layer F.Cu) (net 9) (status 10))
 (segment (start 95.59 118.45) (end 94.94 118.45) (width 0.25) (layer F.Cu) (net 15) (status 30))
 (segment (start 112.014 122.301) (end 112.014 126.365) (width 0.25) (layer F.Cu) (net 15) (status 20))
 (segment (start 111.506 121.793) (end 112.014 122.301) (width 0.25) (layer F.Cu) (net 15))
 (segment (start 107.315 121.412) (end 107.696 121.793) (width 0.25) (layer F.Cu) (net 15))
 (segment (start 104.902 121.412) (end 107.315 121.412) (width 0.25) (layer F.Cu) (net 15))
 (segment (start 98.552 115.57) (end 98.93249 115.95049) (width 0.25) (layer F.Cu) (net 15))
 (segment (start 98.93249 117.321484) (end 100.737006 119.126) (width 0.25) (layer F.Cu) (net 15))
 (segment (start 98.93249 115.95049) (end 98.93249 117.321484) (width 0.25) (layer F.Cu) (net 15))
 (segment (start 100.737006 119.126) (end 103.759 119.126) (width 0.25) (layer F.Cu) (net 15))
 (segment (start 95.59 117.135) (end 97.155 115.57) (width 0.25) (layer F.Cu) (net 15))
 (segment (start 103.759 119.126) (end 104.267 119.634) (width 0.25) (layer F.Cu) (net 15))
 (segment (start 104.267 119.634) (end 104.267 120.777) (width 0.25) (layer F.Cu) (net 15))
 (segment (start 107.696 121.793) (end 111.506 121.793) (width 0.25) (layer F.Cu) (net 15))
 (segment (start 97.155 115.57) (end 98.552 115.57) (width 0.25) (layer F.Cu) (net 15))
 (segment (start 95.59 118.45) (end 95.59 117.135) (width 0.25) (layer F.Cu) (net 15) (status 10))
 (segment (start 104.267 120.777) (end 104.902 121.412) (width 0.25) (layer F.Cu) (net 15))
 (segment (start 85.725 121.41) (end 85.725 123.19) (width 0.25) (layer F.Cu) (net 6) (status 30))
 (segment (start 90.0175 126.1875) (end 90.0175 126.365) (width 0.25) (layer F.Cu) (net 1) (status 30))
 (segment (start 91.745 124.46) (end 90.0175 126.1875) (width 0.25) (layer F.Cu) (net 1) (status 30))
 (segment (start 91.745 124.46) (end 94.869 124.46) (width 0.25) (layer F.Cu) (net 1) (status 10))
 (segment (start 94.869 124.46) (end 95.631 125.222) (width 0.25) (layer F.Cu) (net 1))
 (segment (start 95.631 125.222) (end 95.631 127) (width 0.25) (layer F.Cu) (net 1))
 (segment (start 96.52 127.889) (end 96.52 129.54) (width 0.25) (layer F.Cu) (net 1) (status 20))
 (segment (start 95.631 127) (end 96.52 127.889) (width 0.25) (layer F.Cu) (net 1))
 (segment (start 93.98 125.855) (end 93.855 125.73) (width 0.25) (layer F.Cu) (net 8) (status 30))
 (segment (start 93.98 129.54) (end 93.98 125.855) (width 0.25) (layer F.Cu) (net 8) (status 30))
 (via (at 90.17 114.3) (size 0.8) (drill 0.4) (layers F.Cu B.Cu) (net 8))
 (segment (start 92.405 114.3) (end 90.17 114.3) (width 0.25) (layer F.Cu) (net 8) (status 10))
 (segment (start 92.71 130.81) (end 93.98 129.54) (width 0.25) (layer B.Cu) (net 8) (status 20))
 (segment (start 90.17 114.3) (end 88.9 115.57) (width 0.25) (layer B.Cu) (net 8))
 (segment (start 88.9 115.57) (end 88.9 128.27) (width 0.25) (layer B.Cu) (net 8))
 (segment (start 88.9 128.27) (end 91.44 130.81) (width 0.25) (layer B.Cu) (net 8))
 (segment (start 91.44 130.81) (end 92.71 130.81) (width 0.25) (layer B.Cu) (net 8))
 (segment (start 112.014 128.829) (end 112.09 128.905) (width 0.25) (layer F.Cu) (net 17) (status 30))
 (segment (start 108.204 128.33) (end 108.899 127.635) (width 0.25) (layer F.Cu) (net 17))
 (segment (start 108.204 128.905) (end 108.204 128.33) (width 0.25) (layer F.Cu) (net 17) (status 10))
 (segment (start 110.82 127.635) (end 112.09 128.905) (width 0.25) (layer F.Cu) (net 17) (status 20))
 (segment (start 108.899 127.635) (end 110.82 127.635) (width 0.25) (layer F.Cu) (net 17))
 (segment (start 105.41 127.635) (end 103.505 127.635) (width 0.25) (layer F.Cu) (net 17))
 (segment (start 103.505 127.635) (end 101.6 129.54) (width 0.25) (layer F.Cu) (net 17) (status 20))
 (segment (start 106.68 128.905) (end 105.41 127.635) (width 0.25) (layer F.Cu) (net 17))
 (segment (start 108.204 128.905) (end 106.68 128.905) (width 0.25) (layer F.Cu) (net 17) (status 10))
 (segment (start 95.25 114.3) (end 93.98 114.3) (width 0.25) (layer F.Cu) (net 18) (status 20))
 (segment (start 97.79 111.76) (end 95.25 114.3) (width 0.25) (layer F.Cu) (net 18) (status 10))
 (segment (start 100.33 111.76) (end 106.68 111.76) (width 0.25) (layer B.Cu) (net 20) (status 10))
 (segment (start 106.68 111.76) (end 113.03 118.11) (width 0.25) (layer B.Cu) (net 20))
 (segment (start 113.03 118.11) (end 113.03 129.54) (width 0.25) (layer B.Cu) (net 20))
 (segment (start 113.03 129.54) (end 111.76 130.81) (width 0.25) (layer B.Cu) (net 20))
 (segment (start 111.76 130.81) (end 105.41 130.81) (width 0.25) (layer B.Cu) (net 20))
 (segment (start 105.41 130.81) (end 104.14 129.54) (width 0.25) (layer B.Cu) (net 20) (status 20))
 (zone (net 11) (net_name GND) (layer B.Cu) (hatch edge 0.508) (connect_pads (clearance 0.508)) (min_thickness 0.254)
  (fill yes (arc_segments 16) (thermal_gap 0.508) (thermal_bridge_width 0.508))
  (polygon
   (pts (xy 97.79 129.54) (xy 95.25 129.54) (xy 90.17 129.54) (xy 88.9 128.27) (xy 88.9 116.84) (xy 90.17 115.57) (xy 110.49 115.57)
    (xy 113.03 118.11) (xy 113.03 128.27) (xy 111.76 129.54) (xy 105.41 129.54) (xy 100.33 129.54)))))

